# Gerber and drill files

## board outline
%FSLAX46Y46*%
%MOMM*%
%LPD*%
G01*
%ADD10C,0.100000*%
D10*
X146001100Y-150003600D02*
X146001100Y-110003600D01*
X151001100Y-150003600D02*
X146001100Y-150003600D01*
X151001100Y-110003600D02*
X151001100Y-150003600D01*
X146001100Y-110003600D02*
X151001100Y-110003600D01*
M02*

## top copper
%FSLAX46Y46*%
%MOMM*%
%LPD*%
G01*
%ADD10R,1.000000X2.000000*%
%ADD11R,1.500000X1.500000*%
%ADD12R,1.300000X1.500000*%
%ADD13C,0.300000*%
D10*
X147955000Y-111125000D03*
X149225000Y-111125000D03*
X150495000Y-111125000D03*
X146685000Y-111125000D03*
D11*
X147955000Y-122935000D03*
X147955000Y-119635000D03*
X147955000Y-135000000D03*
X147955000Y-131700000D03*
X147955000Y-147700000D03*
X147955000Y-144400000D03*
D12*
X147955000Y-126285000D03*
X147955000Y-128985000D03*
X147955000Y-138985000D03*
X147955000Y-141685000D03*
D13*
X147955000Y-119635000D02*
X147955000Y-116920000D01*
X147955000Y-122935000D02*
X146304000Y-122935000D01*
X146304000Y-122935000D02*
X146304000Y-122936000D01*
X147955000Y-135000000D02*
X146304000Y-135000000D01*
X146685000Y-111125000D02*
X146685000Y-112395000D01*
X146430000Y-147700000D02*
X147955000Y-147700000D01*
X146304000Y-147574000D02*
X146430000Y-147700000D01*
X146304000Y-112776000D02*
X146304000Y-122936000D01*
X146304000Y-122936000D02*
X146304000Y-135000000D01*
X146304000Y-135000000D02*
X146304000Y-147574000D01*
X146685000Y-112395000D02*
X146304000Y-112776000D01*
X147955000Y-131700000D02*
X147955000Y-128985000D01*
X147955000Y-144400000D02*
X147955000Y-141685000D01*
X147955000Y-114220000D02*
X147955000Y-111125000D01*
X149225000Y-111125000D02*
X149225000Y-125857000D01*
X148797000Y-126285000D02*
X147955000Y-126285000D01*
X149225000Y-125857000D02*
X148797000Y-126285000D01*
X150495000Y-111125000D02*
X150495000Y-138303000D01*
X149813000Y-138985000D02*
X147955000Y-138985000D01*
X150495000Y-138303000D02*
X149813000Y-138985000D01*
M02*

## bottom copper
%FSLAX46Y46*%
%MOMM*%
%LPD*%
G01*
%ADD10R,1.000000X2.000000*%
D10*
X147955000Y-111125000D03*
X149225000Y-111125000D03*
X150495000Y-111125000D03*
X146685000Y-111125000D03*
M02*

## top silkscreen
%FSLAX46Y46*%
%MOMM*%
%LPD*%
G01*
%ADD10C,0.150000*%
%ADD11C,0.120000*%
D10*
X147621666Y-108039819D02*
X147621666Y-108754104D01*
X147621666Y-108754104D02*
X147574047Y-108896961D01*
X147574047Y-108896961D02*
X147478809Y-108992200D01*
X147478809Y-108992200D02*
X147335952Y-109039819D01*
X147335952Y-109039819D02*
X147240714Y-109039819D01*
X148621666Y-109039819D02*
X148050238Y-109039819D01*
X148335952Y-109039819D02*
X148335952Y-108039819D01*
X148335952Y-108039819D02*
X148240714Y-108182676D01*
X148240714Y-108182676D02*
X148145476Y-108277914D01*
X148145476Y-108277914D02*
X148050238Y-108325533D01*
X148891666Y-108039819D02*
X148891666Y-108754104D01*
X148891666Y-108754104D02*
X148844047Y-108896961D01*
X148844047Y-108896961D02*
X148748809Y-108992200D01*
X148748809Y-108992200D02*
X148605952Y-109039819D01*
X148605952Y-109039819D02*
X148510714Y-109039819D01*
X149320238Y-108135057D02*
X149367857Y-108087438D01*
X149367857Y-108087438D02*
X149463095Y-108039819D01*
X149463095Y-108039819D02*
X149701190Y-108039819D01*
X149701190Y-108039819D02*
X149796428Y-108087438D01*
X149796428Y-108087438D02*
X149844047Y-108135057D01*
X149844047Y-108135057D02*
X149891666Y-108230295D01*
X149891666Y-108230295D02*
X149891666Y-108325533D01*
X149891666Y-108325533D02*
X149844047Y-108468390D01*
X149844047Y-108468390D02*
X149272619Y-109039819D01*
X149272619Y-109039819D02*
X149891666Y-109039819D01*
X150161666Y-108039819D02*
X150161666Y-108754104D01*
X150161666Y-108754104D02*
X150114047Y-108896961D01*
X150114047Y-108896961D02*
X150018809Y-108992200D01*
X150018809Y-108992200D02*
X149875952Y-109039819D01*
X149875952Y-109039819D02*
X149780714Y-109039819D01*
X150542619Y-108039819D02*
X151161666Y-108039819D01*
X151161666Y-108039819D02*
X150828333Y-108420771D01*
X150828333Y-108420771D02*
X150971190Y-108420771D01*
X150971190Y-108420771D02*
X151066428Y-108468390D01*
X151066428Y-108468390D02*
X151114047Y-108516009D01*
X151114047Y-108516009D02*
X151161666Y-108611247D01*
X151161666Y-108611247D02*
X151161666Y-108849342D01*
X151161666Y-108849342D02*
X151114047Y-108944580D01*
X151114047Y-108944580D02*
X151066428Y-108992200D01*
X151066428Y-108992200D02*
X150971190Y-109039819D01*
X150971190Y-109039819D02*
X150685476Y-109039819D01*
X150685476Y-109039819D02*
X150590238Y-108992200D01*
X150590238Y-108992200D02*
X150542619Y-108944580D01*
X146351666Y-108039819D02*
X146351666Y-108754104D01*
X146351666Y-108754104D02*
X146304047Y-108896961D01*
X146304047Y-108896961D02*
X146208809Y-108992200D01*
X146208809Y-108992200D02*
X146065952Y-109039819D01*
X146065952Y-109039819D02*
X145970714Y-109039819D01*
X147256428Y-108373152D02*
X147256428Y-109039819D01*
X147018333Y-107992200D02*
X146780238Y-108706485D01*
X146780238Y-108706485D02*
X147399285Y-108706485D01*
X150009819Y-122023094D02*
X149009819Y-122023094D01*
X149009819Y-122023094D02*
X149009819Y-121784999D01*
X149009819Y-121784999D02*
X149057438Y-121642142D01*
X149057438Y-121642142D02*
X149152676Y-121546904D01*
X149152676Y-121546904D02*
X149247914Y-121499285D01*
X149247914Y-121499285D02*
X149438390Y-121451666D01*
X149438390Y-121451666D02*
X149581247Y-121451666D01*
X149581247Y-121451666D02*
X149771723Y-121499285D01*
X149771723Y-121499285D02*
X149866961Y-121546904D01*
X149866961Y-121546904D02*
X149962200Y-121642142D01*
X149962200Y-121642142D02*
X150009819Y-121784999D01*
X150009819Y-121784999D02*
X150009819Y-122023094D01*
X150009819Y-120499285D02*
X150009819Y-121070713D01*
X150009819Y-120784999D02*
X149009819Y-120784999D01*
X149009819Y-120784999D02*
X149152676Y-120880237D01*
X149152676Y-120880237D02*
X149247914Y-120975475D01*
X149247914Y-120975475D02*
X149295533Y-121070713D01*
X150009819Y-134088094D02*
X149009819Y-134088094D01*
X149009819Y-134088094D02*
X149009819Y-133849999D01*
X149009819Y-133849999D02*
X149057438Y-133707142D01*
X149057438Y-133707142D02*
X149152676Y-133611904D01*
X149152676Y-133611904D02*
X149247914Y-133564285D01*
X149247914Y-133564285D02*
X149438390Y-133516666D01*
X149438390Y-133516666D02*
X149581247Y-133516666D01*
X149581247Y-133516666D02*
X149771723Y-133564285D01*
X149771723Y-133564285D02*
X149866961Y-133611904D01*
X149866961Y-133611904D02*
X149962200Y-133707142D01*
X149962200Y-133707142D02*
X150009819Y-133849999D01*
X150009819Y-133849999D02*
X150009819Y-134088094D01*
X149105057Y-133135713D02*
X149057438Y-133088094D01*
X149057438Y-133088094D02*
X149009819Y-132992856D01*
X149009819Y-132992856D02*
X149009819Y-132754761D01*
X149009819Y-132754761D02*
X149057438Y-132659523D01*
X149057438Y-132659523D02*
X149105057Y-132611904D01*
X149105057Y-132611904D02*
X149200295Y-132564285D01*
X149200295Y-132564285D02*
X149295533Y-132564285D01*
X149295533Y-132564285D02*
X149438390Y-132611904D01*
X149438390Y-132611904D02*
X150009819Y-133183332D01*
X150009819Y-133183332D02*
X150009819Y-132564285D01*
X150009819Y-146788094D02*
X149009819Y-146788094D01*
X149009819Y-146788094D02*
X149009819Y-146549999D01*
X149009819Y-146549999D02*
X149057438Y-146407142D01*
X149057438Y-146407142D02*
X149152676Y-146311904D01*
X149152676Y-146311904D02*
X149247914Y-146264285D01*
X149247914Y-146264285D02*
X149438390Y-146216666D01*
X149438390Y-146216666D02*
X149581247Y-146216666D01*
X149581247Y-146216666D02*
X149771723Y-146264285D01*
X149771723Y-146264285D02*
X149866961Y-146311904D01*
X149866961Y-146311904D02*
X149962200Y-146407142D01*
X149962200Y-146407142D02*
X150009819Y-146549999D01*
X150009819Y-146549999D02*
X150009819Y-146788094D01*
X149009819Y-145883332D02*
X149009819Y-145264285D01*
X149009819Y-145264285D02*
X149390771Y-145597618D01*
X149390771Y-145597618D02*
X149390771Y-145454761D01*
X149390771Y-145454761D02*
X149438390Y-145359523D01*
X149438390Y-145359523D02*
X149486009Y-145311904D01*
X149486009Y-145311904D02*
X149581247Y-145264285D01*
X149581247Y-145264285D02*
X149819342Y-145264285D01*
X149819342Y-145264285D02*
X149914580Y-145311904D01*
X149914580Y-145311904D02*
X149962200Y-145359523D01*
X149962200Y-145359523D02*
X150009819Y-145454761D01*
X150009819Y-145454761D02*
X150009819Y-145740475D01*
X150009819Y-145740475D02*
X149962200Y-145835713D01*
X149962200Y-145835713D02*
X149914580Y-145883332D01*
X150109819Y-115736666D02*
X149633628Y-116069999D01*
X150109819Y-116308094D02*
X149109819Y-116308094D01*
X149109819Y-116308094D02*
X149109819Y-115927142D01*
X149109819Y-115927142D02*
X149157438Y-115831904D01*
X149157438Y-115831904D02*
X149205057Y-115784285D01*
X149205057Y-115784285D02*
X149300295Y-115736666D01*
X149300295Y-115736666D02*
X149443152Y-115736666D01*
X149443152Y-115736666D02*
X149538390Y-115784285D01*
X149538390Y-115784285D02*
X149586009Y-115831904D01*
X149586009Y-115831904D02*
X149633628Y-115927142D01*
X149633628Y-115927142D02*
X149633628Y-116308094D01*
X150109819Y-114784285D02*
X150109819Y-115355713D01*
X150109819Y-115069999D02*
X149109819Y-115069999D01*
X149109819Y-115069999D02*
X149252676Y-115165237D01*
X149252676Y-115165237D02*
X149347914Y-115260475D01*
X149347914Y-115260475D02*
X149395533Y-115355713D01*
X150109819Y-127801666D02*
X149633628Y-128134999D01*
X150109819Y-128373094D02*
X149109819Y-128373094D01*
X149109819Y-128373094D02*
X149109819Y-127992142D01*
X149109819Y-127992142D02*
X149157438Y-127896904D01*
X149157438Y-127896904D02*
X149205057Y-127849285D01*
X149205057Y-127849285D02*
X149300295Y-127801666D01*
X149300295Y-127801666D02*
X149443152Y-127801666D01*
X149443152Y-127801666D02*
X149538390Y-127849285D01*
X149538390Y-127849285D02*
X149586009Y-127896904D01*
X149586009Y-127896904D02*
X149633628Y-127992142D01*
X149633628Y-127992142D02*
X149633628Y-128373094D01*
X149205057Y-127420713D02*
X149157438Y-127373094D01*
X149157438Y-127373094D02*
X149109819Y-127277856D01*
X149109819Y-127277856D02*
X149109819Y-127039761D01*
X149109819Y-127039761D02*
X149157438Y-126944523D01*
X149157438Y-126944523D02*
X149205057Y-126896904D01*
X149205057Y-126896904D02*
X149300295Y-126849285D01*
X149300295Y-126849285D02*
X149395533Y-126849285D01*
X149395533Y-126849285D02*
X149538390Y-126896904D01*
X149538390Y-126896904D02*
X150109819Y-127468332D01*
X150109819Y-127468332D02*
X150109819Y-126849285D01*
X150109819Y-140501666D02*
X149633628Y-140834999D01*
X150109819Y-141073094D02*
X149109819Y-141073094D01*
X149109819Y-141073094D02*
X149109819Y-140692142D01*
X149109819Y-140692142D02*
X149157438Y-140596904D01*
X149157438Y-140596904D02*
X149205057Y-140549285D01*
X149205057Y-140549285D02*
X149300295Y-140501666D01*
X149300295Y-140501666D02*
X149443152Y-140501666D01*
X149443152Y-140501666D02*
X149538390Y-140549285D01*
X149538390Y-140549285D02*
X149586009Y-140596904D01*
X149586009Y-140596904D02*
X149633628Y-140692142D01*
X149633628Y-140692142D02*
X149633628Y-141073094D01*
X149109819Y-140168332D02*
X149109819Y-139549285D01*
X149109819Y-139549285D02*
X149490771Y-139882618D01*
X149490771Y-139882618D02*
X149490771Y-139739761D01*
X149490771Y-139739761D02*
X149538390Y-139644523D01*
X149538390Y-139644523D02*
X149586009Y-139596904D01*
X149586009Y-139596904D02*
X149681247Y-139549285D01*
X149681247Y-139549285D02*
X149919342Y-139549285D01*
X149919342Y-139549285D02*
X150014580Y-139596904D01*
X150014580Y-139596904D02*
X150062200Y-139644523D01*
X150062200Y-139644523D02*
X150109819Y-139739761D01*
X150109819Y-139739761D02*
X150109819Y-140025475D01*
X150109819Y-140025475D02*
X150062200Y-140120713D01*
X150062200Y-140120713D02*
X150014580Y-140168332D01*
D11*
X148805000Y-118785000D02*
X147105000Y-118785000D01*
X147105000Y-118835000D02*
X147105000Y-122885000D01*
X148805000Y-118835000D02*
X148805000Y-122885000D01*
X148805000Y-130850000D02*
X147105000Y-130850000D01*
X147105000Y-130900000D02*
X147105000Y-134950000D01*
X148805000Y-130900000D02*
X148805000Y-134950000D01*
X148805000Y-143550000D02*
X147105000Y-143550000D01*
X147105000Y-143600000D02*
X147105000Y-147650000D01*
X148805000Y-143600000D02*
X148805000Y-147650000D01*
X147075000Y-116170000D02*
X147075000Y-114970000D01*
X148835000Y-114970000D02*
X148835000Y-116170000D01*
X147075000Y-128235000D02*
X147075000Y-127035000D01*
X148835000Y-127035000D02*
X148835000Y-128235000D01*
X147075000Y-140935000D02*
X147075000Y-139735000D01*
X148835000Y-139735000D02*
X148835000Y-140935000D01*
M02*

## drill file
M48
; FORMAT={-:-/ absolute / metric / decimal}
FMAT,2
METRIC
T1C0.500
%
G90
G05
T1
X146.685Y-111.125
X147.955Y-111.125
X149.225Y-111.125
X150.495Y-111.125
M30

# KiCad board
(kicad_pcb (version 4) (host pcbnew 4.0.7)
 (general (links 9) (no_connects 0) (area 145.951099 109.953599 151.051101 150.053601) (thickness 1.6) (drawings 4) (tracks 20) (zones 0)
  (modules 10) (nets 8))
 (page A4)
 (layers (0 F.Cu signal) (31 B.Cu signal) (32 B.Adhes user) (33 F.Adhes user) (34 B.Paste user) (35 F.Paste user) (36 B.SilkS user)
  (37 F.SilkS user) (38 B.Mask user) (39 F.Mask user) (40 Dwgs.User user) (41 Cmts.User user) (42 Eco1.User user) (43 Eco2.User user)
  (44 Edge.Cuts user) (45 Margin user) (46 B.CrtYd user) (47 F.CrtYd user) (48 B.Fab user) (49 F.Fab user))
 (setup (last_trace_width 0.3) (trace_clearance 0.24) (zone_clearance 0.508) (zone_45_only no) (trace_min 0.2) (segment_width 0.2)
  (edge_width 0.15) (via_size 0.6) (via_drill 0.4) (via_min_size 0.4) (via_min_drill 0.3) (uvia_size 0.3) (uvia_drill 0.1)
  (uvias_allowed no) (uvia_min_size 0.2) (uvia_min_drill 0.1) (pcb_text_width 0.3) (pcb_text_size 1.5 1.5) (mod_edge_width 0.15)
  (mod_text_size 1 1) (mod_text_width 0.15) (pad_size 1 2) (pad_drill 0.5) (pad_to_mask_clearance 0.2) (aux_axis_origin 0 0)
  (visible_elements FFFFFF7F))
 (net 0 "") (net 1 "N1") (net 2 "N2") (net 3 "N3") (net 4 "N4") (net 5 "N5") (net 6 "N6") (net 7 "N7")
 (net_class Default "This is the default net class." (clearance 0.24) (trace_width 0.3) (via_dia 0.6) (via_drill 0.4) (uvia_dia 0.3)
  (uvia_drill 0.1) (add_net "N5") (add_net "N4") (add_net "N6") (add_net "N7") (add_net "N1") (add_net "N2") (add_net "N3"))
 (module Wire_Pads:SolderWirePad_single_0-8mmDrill (layer F.Cu) (at 147.955 111.125)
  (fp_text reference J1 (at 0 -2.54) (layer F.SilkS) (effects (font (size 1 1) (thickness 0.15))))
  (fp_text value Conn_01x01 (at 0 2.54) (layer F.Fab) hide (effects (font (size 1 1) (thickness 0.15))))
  (pad 1 thru_hole rect (at 0 0) (size 1 2) (drill 0.5) (layers *.Cu *.Mask) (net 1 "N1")))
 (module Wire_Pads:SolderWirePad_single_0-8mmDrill (layer F.Cu) (at 149.225 111.125)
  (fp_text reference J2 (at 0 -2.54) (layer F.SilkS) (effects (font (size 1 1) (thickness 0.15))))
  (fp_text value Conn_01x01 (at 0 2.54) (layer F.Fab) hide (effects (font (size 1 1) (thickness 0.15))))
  (pad 1 thru_hole rect (at 0 0) (size 1 2) (drill 0.5) (layers *.Cu *.Mask) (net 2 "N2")))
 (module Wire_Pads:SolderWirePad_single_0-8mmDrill (layer F.Cu) (at 150.495 111.125)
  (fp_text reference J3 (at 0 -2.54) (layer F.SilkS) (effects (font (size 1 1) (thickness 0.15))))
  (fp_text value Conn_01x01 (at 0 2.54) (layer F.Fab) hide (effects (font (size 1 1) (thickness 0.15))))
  (pad 1 thru_hole rect (at 0 0) (size 1 2) (drill 0.5) (layers *.Cu *.Mask) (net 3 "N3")))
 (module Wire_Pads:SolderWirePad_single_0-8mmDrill (layer F.Cu) (at 146.685 111.125)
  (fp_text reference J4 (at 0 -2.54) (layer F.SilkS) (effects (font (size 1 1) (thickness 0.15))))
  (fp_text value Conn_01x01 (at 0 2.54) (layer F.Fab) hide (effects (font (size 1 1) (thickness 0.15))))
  (pad 1 thru_hole rect (at 0 0) (size 1 2) (drill 0.5) (layers *.Cu *.Mask) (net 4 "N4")))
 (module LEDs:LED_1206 (layer F.Cu) (at 147.955 121.285 270)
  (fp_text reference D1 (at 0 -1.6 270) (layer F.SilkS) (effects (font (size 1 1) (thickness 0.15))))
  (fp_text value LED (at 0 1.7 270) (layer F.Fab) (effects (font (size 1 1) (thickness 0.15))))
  (fp_line (start -2.5 -0.85) (end -2.5 0.85) (layer F.SilkS) (width 0.12))
  (fp_line (start -2.45 0.85) (end 1.6 0.85) (layer F.SilkS) (width 0.12))
  (fp_line (start -2.45 -0.85) (end 1.6 -0.85) (layer F.SilkS) (width 0.12))
  (pad 2 smd rect (at 1.65 0 90) (size 1.5 1.5) (layers F.Cu F.Paste F.Mask) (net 4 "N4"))
  (pad 1 smd rect (at -1.65 0 90) (size 1.5 1.5) (layers F.Cu F.Paste F.Mask) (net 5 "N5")))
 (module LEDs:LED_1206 (layer F.Cu) (at 147.955 133.35 270)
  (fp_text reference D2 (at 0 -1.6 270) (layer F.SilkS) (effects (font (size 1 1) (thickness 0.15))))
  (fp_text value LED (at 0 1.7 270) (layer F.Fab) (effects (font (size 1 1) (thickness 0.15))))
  (fp_line (start -2.5 -0.85) (end -2.5 0.85) (layer F.SilkS) (width 0.12))
  (fp_line (start -2.45 0.85) (end 1.6 0.85) (layer F.SilkS) (width 0.12))
  (fp_line (start -2.45 -0.85) (end 1.6 -0.85) (layer F.SilkS) (width 0.12))
  (pad 2 smd rect (at 1.65 0 90) (size 1.5 1.5) (layers F.Cu F.Paste F.Mask) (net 4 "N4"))
  (pad 1 smd rect (at -1.65 0 90) (size 1.5 1.5) (layers F.Cu F.Paste F.Mask) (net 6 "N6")))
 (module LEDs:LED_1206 (layer F.Cu) (at 147.955 146.05 270)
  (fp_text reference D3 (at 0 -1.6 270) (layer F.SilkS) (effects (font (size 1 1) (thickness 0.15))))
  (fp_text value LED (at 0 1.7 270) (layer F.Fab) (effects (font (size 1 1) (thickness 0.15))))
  (fp_line (start -2.5 -0.85) (end -2.5 0.85) (layer F.SilkS) (width 0.12))
  (fp_line (start -2.45 0.85) (end 1.6 0.85) (layer F.SilkS) (width 0.12))
  (fp_line (start -2.45 -0.85) (end 1.6 -0.85) (layer F.SilkS) (width 0.12))
  (pad 2 smd rect (at 1.65 0 90) (size 1.5 1.5) (layers F.Cu F.Paste F.Mask) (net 4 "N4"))
  (pad 1 smd rect (at -1.65 0 90) (size 1.5 1.5) (layers F.Cu F.Paste F.Mask) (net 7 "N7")))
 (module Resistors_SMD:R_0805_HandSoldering (layer F.Cu) (at 147.955 115.57 270)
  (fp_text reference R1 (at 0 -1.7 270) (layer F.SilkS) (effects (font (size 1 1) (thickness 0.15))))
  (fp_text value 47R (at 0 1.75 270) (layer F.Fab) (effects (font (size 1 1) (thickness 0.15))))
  (fp_line (start 0.6 0.88) (end -0.6 0.88) (layer F.SilkS) (width 0.12))
  (fp_line (start -0.6 -0.88) (end 0.6 -0.88) (layer F.SilkS) (width 0.12)))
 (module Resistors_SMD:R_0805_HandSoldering (layer F.Cu) (at 147.955 127.635 270)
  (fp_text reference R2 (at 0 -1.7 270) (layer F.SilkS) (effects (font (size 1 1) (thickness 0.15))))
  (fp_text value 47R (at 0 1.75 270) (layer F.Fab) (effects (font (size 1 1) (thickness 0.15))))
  (fp_line (start 0.6 0.88) (end -0.6 0.88) (layer F.SilkS) (width 0.12))
  (fp_line (start -0.6 -0.88) (end 0.6 -0.88) (layer F.SilkS) (width 0.12))
  (pad 1 smd rect (at -1.35 0 270) (size 1.5 1.3) (layers F.Cu F.Paste F.Mask) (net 2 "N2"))
  (pad 2 smd rect (at 1.35 0 270) (size 1.5 1.3) (layers F.Cu F.Paste F.Mask) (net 6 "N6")))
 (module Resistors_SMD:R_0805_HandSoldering (layer F.Cu) (at 147.955 140.335 270)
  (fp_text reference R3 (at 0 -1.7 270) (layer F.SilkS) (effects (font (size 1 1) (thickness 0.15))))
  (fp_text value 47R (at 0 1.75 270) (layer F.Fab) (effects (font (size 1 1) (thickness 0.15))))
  (fp_line (start 0.6 0.88) (end -0.6 0.88) (layer F.SilkS) (width 0.12))
  (fp_line (start -0.6 -0.88) (end 0.6 -0.88) (layer F.SilkS) (width 0.12))
  (pad 1 smd rect (at -1.35 0 270) (size 1.5 1.3) (layers F.Cu F.Paste F.Mask) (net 3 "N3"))
  (pad 2 smd rect (at 1.35 0 270) (size 1.5 1.3) (layers F.Cu F.Paste F.Mask) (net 7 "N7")))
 (gr_line (start 146.0011 150.0036) (end 146.0011 110.0036) (layer Edge.Cuts) (width 0.1))
 (gr_line (start 151.0011 150.0036) (end 146.0011 150.0036) (layer Edge.Cuts) (width 0.1))
 (gr_line (start 151.0011 110.0036) (end 151.0011 150.0036) (layer Edge.Cuts) (width 0.1))
 (gr_line (start 146.0011 110.0036) (end 151.0011 110.0036) (layer Edge.Cuts) (width 0.1))
 (segment (start 147.955 119.635) (end 147.955 116.92) (width 0.3) (layer F.Cu) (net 5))
 (segment (start 147.955 122.935) (end 146.304 122.935) (width 0.3) (layer F.Cu) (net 4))
 (segment (start 146.304 122.935) (end 146.304 122.936) (width 0.3) (layer F.Cu) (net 4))
 (segment (start 147.955 135) (end 146.304 135) (width 0.3) (layer F.Cu) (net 4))
 (segment (start 146.685 111.125) (end 146.685 112.395) (width 0.3) (layer F.Cu) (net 4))
 (segment (start 146.43 147.7) (end 147.955 147.7) (width 0.3) (layer F.Cu) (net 4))
 (segment (start 146.304 147.574) (end 146.43 147.7) (width 0.3) (layer F.Cu) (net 4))
 (segment (start 146.304 112.776) (end 146.304 122.936) (width 0.3) (layer F.Cu) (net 4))
 (segment (start 146.304 122.936) (end 146.304 135) (width 0.3) (layer F.Cu) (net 4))
 (segment (start 146.304 135) (end 146.304 147.574) (width 0.3) (layer F.Cu) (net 4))
 (segment (start 146.685 112.395) (end 146.304 112.776) (width 0.3) (layer F.Cu) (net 4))
 (segment (start 147.955 131.7) (end 147.955 128.985) (width 0.3) (layer F.Cu) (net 6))
 (segment (start 147.955 144.4) (end 147.955 141.685) (width 0.3) (layer F.Cu) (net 7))
 (segment (start 147.955 114.22) (end 147.955 111.125) (width 0.3) (layer F.Cu) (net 1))
 (segment (start 149.225 111.125) (end 149.225 125.857) (width 0.3) (layer F.Cu) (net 2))
 (segment (start 148.797 126.285) (end 147.955 126.285) (width 0.3) (layer F.Cu) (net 2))
 (segment (start 149.225 125.857) (end 148.797 126.285) (width 0.3) (layer F.Cu) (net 2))
 (segment (start 150.495 111.125) (end 150.495 138.303) (width 0.3) (layer F.Cu) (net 3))
 (segment (start 149.813 138.985) (end 147.955 138.985) (width 0.3) (layer F.Cu) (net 3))
 (segment (start 150.495 138.303) (end 149.813 138.985) (width 0.3) (layer F.Cu) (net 3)))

